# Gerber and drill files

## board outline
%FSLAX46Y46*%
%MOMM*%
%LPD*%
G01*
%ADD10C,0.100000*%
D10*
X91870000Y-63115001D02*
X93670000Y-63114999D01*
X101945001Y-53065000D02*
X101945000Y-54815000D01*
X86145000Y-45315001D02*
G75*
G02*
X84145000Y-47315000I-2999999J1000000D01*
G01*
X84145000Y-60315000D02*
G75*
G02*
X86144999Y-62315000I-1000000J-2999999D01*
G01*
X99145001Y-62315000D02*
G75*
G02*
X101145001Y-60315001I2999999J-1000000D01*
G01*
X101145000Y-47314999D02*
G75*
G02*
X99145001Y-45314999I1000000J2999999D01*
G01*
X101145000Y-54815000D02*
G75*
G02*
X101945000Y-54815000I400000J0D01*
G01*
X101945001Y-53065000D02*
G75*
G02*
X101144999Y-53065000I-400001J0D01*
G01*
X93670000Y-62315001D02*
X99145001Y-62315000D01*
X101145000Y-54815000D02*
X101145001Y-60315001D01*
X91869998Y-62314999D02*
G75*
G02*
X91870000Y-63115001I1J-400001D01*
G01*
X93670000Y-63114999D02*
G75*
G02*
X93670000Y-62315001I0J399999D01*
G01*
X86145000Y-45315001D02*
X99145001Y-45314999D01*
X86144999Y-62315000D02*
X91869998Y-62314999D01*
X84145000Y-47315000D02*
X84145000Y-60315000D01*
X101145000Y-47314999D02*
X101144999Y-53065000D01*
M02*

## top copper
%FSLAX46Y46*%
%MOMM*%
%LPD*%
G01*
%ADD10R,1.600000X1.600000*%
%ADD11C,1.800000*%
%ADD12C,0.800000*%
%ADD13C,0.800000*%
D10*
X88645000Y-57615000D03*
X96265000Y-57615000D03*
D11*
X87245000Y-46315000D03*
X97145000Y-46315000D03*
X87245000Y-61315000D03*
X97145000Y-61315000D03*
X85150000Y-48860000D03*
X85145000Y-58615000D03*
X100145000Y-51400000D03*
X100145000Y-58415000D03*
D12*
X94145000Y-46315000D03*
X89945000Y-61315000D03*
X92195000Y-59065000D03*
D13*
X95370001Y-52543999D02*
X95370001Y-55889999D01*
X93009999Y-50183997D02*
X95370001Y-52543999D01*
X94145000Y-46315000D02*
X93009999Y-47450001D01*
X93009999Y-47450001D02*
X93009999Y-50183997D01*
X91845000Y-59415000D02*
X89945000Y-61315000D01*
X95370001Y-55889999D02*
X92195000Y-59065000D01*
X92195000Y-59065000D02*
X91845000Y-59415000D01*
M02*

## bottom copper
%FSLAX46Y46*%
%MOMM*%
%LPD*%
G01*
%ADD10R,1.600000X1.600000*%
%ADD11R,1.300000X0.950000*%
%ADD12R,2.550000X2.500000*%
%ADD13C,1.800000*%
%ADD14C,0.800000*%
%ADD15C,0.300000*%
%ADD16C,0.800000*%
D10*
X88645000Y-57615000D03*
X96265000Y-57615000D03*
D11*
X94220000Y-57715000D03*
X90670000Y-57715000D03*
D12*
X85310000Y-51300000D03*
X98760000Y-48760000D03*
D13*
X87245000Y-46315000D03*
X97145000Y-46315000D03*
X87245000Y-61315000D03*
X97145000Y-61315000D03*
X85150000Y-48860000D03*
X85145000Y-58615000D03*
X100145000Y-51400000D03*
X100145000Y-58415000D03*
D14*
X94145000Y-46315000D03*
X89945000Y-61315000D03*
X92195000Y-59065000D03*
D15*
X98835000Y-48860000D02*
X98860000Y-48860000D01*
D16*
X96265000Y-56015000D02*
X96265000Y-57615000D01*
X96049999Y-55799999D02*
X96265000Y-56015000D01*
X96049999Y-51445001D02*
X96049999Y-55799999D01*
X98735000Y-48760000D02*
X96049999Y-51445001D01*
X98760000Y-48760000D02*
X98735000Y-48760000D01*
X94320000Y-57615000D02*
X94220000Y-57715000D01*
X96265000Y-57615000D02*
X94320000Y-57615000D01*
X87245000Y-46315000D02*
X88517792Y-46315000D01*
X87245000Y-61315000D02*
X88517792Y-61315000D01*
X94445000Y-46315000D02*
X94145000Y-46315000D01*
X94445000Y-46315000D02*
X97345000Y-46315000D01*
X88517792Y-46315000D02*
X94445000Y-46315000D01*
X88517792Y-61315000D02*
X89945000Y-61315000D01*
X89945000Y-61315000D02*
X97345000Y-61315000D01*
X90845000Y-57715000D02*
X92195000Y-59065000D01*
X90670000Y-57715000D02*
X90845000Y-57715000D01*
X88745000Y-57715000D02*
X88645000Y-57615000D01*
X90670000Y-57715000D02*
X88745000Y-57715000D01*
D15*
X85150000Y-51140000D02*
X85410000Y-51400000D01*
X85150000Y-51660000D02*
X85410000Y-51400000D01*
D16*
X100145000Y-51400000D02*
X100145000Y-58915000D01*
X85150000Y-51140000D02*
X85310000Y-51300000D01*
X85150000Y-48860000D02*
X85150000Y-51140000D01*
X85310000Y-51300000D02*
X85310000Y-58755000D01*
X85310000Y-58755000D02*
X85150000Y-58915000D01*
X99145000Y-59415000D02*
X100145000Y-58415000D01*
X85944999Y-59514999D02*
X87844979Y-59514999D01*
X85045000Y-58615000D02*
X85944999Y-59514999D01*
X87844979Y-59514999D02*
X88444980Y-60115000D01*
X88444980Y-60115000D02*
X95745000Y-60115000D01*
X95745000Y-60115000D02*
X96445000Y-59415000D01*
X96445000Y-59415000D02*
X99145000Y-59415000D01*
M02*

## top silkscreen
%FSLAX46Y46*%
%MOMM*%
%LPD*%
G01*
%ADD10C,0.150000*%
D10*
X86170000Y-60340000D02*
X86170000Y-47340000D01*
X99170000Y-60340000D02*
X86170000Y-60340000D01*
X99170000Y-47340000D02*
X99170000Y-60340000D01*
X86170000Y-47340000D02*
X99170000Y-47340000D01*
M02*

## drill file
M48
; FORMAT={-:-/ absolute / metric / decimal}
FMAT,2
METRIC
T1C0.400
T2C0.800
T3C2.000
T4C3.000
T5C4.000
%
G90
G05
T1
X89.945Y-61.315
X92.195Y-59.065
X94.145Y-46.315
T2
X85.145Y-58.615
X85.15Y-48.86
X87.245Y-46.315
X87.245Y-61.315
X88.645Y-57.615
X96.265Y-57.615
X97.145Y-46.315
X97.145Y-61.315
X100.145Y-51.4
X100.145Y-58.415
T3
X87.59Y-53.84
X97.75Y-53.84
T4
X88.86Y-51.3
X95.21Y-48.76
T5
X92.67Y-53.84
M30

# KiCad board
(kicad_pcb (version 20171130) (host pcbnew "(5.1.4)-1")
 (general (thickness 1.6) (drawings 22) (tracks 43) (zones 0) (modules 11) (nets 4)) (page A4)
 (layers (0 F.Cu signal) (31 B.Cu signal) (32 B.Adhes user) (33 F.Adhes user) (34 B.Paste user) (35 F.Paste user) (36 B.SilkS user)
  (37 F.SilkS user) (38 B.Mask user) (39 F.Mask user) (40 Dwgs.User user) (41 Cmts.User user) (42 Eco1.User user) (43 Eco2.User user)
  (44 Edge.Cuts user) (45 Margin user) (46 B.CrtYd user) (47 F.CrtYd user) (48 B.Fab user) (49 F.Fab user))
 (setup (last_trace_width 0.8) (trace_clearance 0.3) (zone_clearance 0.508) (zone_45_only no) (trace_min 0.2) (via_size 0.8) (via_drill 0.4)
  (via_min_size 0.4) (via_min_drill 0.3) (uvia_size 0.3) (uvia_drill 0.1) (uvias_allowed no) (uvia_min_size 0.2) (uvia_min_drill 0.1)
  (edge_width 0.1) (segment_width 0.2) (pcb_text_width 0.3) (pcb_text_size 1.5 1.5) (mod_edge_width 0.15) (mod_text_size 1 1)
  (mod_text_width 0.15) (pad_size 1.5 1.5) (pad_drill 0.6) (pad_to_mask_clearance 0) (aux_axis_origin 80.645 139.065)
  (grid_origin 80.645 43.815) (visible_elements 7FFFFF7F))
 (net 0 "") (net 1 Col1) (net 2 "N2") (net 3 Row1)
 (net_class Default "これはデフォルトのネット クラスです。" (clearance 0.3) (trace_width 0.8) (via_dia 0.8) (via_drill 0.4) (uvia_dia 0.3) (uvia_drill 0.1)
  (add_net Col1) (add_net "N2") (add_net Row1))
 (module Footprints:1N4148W (layer B.Cu) (at 88.645 57.615)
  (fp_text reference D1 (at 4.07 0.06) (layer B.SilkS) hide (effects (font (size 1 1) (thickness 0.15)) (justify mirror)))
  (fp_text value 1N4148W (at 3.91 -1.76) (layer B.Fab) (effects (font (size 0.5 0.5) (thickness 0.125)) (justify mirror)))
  (pad 1 thru_hole rect (at 0 0) (size 1.6 1.6) (drill 0.8) (layers *.Cu *.Mask) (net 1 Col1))
  (pad 2 thru_hole rect (at 7.62 0) (size 1.6 1.6) (drill 0.8) (layers *.Cu *.Mask) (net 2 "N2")))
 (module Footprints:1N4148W (layer B.Cu) (at 92.445 57.715)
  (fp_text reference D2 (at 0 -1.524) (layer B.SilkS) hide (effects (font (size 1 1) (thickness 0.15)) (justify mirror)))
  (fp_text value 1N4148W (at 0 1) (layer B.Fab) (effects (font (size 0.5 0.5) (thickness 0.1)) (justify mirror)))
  (pad 2 smd rect (at 1.775 0) (size 1.3 0.95) (layers B.Cu B.Paste B.Mask) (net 2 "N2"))
  (pad 1 smd rect (at -1.775 0) (size 1.3 0.95) (layers B.Cu B.Paste B.Mask) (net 1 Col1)))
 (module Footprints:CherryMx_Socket (layer F.Cu) (at 92.67 53.84)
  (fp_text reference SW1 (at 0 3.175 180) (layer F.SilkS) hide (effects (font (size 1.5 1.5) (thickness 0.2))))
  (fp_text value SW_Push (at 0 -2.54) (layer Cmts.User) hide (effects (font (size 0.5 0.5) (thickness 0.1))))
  (fp_line (start -6.5 6.5) (end -6.5 -6.5) (layer F.SilkS) (width 0.15))
  (fp_line (start 6.5 6.5) (end -6.5 6.5) (layer F.SilkS) (width 0.15))
  (fp_line (start 6.5 -6.5) (end 6.5 6.5) (layer F.SilkS) (width 0.15))
  (fp_line (start -6.5 -6.5) (end 6.5 -6.5) (layer F.SilkS) (width 0.15))
  (pad 1 smd rect (at -7.36 -2.54) (size 2.55 2.5) (layers B.Cu B.Paste B.Mask) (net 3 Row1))
  (pad 2 smd rect (at 6.09 -5.08) (size 2.55 2.5) (layers B.Cu B.Paste B.Mask) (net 2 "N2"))
  (pad "" np_thru_hole circle (at -5.08 0) (size 2 2) (drill 2) (layers *.Cu *.Mask))
  (pad "" np_thru_hole circle (at -3.81 -2.54) (size 3 3) (drill 3) (layers *.Cu *.Mask))
  (pad "" np_thru_hole circle (at 0 0) (size 4 4) (drill 4) (layers *.Cu *.Mask))
  (pad "" np_thru_hole circle (at 2.54 -5.08) (size 3 3) (drill 3) (layers *.Cu *.Mask))
  (pad "" np_thru_hole circle (at 5.08 0) (size 2 2) (drill 2) (layers *.Cu *.Mask)))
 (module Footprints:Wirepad (layer B.Cu) (at 87.245 46.315)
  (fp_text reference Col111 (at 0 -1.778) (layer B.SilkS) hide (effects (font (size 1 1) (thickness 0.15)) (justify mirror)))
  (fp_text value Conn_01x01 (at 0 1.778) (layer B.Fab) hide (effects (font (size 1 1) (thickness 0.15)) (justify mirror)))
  (pad 1 thru_hole circle (at 0 0) (size 1.8 1.8) (drill 0.8) (layers B.Cu B.Mask) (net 1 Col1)))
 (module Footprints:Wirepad (layer B.Cu) (at 97.145 46.315)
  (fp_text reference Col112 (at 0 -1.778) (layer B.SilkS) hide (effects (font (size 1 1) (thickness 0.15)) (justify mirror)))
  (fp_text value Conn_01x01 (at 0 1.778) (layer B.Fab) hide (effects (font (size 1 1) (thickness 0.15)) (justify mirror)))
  (pad 1 thru_hole circle (at 0 0) (size 1.8 1.8) (drill 0.8) (layers B.Cu B.Mask) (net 1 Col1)))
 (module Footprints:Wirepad (layer B.Cu) (at 87.245 61.315)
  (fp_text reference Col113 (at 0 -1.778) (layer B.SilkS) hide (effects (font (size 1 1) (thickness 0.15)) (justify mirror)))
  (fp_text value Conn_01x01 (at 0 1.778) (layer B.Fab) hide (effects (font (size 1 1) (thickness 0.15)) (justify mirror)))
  (pad 1 thru_hole circle (at 0 0) (size 1.8 1.8) (drill 0.8) (layers B.Cu B.Mask) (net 1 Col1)))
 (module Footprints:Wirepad (layer B.Cu) (at 97.145 61.315)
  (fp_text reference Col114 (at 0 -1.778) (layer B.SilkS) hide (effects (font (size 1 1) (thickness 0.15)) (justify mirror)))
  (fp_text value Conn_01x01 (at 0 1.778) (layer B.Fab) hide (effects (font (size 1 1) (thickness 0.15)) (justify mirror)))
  (pad 1 thru_hole circle (at 0 0) (size 1.8 1.8) (drill 0.8) (layers B.Cu B.Mask) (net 1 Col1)))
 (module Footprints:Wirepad (layer B.Cu) (at 85.15 48.86)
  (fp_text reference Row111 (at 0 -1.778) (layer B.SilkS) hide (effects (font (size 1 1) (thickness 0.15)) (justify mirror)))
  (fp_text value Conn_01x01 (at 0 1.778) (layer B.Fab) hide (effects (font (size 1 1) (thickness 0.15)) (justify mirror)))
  (pad 1 thru_hole circle (at 0 0) (size 1.8 1.8) (drill 0.8) (layers B.Cu B.Mask) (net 3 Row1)))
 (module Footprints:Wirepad (layer B.Cu) (at 85.145 58.615)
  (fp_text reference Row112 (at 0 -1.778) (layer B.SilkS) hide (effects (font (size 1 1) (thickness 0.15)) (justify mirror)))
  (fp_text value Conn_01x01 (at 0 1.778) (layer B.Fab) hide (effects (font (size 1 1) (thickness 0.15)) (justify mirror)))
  (pad 1 thru_hole circle (at 0 0) (size 1.8 1.8) (drill 0.8) (layers B.Cu B.Mask) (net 3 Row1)))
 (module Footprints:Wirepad (layer B.Cu) (at 100.145 51.4)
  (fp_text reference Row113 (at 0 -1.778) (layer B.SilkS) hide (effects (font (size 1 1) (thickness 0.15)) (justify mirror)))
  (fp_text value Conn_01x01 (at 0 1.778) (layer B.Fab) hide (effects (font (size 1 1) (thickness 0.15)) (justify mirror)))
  (pad 1 thru_hole circle (at 0 0) (size 1.8 1.8) (drill 0.8) (layers B.Cu B.Mask) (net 3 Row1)))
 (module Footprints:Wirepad (layer B.Cu) (at 100.145 58.415)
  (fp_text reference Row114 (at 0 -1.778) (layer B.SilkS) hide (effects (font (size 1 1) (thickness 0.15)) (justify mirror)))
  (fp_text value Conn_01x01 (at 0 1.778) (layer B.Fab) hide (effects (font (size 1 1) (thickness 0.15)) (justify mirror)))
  (pad 1 thru_hole circle (at 0 0) (size 1.8 1.8) (drill 0.8) (layers B.Cu B.Mask) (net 3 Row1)))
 (gr_line (start 91.87 63.115001) (end 93.67 63.114999) (layer Edge.Cuts) (width 0.1))
 (gr_line (start 101.945001 53.065) (end 101.945 54.815) (layer Edge.Cuts) (width 0.1))
 (gr_arc (start 83.145001 44.315001) (end 84.145 47.315) (angle -53.13010235) (layer Edge.Cuts) (width 0.1))
 (gr_arc (start 83.145 63.314999) (end 86.144999 62.315) (angle -53.13010235) (layer Edge.Cuts) (width 0.1))
 (gr_arc (start 102.145 63.315) (end 101.145001 60.315001) (angle -53.13010235) (layer Edge.Cuts) (width 0.1))
 (gr_arc (start 102.145 44.315) (end 99.145001 45.314999) (angle -53.13010235) (layer Edge.Cuts) (width 0.1))
 (gr_arc (start 101.545 54.815) (end 101.945 54.815) (angle -180) (layer Edge.Cuts) (width 0.1))
 (gr_arc (start 101.545 53.065) (end 101.144999 53.065) (angle -180) (layer Edge.Cuts) (width 0.1))
 (gr_line (start 93.67 62.315001) (end 99.145001 62.315) (layer Edge.Cuts) (width 0.1))
 (gr_line (start 101.145 54.815) (end 101.145001 60.315001) (layer Edge.Cuts) (width 0.1))
 (gr_arc (start 91.869999 62.715) (end 91.87 63.115001) (angle -180) (layer Edge.Cuts) (width 0.1))
 (gr_arc (start 93.67 62.715) (end 93.67 62.315001) (angle -180) (layer Edge.Cuts) (width 0.1))
 (gr_line (start 86.145 45.315001) (end 99.145001 45.314999) (layer Edge.Cuts) (width 0.1))
 (gr_line (start 86.144999 62.315) (end 91.869998 62.314999) (layer Edge.Cuts) (width 0.1))
 (gr_line (start 84.145 47.315) (end 84.145 60.315) (layer Edge.Cuts) (width 0.1))
 (gr_line (start 101.145 47.314999) (end 101.144999 53.065) (layer Edge.Cuts) (width 0.1))
 (segment (start 98.835 48.86) (end 98.86 48.86) (width 0.3) (layer B.Cu) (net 2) (status 30))
 (segment (start 96.265 56.015) (end 96.265 57.615) (width 0.8) (layer B.Cu) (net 2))
 (segment (start 96.049999 55.799999) (end 96.265 56.015) (width 0.8) (layer B.Cu) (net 2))
 (segment (start 96.049999 51.445001) (end 96.049999 55.799999) (width 0.8) (layer B.Cu) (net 2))
 (segment (start 98.735 48.76) (end 96.049999 51.445001) (width 0.8) (layer B.Cu) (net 2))
 (segment (start 98.76 48.76) (end 98.735 48.76) (width 0.8) (layer B.Cu) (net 2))
 (segment (start 94.32 57.615) (end 94.22 57.715) (width 0.8) (layer B.Cu) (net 2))
 (segment (start 96.265 57.615) (end 94.32 57.615) (width 0.8) (layer B.Cu) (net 2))
 (segment (start 87.245 46.315) (end 88.517792 46.315) (width 0.8) (layer B.Cu) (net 1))
 (segment (start 87.245 61.315) (end 88.517792 61.315) (width 0.8) (layer B.Cu) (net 1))
 (via (at 94.145 46.315) (size 0.8) (drill 0.4) (layers F.Cu B.Cu) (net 1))
 (segment (start 94.445 46.315) (end 94.145 46.315) (width 0.8) (layer B.Cu) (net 1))
 (segment (start 94.445 46.315) (end 97.345 46.315) (width 0.8) (layer B.Cu) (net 1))
 (segment (start 88.517792 46.315) (end 94.445 46.315) (width 0.8) (layer B.Cu) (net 1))
 (segment (start 95.370001 52.543999) (end 95.370001 55.889999) (width 0.8) (layer F.Cu) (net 1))
 (segment (start 93.009999 50.183997) (end 95.370001 52.543999) (width 0.8) (layer F.Cu) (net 1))
 (segment (start 94.145 46.315) (end 93.009999 47.450001) (width 0.8) (layer F.Cu) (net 1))
 (segment (start 93.009999 47.450001) (end 93.009999 50.183997) (width 0.8) (layer F.Cu) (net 1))
 (via (at 89.945 61.315) (size 0.8) (drill 0.4) (layers F.Cu B.Cu) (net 1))
 (segment (start 91.845 59.415) (end 89.945 61.315) (width 0.8) (layer F.Cu) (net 1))
 (segment (start 88.517792 61.315) (end 89.945 61.315) (width 0.8) (layer B.Cu) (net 1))
 (segment (start 89.945 61.315) (end 97.345 61.315) (width 0.8) (layer B.Cu) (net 1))
 (via (at 92.195 59.065) (size 0.8) (drill 0.4) (layers F.Cu B.Cu) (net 1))
 (segment (start 90.845 57.715) (end 92.195 59.065) (width 0.8) (layer B.Cu) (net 1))
 (segment (start 90.67 57.715) (end 90.845 57.715) (width 0.8) (layer B.Cu) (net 1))
 (segment (start 95.370001 55.889999) (end 92.195 59.065) (width 0.8) (layer F.Cu) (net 1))
 (segment (start 92.195 59.065) (end 91.845 59.415) (width 0.8) (layer F.Cu) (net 1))
 (segment (start 88.745 57.715) (end 88.645 57.615) (width 0.8) (layer B.Cu) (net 1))
 (segment (start 90.67 57.715) (end 88.745 57.715) (width 0.8) (layer B.Cu) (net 1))
 (segment (start 85.15 51.14) (end 85.41 51.4) (width 0.3) (layer B.Cu) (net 3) (status 30))
 (segment (start 85.15 51.66) (end 85.41 51.4) (width 0.3) (layer B.Cu) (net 3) (status 30))
 (segment (start 100.145 51.4) (end 100.145 58.915) (width 0.8) (layer B.Cu) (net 3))
 (segment (start 85.15 51.14) (end 85.31 51.3) (width 0.8) (layer B.Cu) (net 3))
 (segment (start 85.15 48.86) (end 85.15 51.14) (width 0.8) (layer B.Cu) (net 3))
 (segment (start 85.31 51.3) (end 85.31 58.755) (width 0.8) (layer B.Cu) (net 3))
 (segment (start 85.31 58.755) (end 85.15 58.915) (width 0.8) (layer B.Cu) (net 3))
 (segment (start 99.145 59.415) (end 100.145 58.415) (width 0.8) (layer B.Cu) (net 3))
 (segment (start 85.944999 59.514999) (end 87.844979 59.514999) (width 0.8) (layer B.Cu) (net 3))
 (segment (start 85.045 58.615) (end 85.944999 59.514999) (width 0.8) (layer B.Cu) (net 3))
 (segment (start 87.844979 59.514999) (end 88.44498 60.115) (width 0.8) (layer B.Cu) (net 3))
 (segment (start 88.44498 60.115) (end 95.745 60.115) (width 0.8) (layer B.Cu) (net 3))
 (segment (start 95.745 60.115) (end 96.445 59.415) (width 0.8) (layer B.Cu) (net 3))
 (segment (start 96.445 59.415) (end 99.145 59.415) (width 0.8) (layer B.Cu) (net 3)))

